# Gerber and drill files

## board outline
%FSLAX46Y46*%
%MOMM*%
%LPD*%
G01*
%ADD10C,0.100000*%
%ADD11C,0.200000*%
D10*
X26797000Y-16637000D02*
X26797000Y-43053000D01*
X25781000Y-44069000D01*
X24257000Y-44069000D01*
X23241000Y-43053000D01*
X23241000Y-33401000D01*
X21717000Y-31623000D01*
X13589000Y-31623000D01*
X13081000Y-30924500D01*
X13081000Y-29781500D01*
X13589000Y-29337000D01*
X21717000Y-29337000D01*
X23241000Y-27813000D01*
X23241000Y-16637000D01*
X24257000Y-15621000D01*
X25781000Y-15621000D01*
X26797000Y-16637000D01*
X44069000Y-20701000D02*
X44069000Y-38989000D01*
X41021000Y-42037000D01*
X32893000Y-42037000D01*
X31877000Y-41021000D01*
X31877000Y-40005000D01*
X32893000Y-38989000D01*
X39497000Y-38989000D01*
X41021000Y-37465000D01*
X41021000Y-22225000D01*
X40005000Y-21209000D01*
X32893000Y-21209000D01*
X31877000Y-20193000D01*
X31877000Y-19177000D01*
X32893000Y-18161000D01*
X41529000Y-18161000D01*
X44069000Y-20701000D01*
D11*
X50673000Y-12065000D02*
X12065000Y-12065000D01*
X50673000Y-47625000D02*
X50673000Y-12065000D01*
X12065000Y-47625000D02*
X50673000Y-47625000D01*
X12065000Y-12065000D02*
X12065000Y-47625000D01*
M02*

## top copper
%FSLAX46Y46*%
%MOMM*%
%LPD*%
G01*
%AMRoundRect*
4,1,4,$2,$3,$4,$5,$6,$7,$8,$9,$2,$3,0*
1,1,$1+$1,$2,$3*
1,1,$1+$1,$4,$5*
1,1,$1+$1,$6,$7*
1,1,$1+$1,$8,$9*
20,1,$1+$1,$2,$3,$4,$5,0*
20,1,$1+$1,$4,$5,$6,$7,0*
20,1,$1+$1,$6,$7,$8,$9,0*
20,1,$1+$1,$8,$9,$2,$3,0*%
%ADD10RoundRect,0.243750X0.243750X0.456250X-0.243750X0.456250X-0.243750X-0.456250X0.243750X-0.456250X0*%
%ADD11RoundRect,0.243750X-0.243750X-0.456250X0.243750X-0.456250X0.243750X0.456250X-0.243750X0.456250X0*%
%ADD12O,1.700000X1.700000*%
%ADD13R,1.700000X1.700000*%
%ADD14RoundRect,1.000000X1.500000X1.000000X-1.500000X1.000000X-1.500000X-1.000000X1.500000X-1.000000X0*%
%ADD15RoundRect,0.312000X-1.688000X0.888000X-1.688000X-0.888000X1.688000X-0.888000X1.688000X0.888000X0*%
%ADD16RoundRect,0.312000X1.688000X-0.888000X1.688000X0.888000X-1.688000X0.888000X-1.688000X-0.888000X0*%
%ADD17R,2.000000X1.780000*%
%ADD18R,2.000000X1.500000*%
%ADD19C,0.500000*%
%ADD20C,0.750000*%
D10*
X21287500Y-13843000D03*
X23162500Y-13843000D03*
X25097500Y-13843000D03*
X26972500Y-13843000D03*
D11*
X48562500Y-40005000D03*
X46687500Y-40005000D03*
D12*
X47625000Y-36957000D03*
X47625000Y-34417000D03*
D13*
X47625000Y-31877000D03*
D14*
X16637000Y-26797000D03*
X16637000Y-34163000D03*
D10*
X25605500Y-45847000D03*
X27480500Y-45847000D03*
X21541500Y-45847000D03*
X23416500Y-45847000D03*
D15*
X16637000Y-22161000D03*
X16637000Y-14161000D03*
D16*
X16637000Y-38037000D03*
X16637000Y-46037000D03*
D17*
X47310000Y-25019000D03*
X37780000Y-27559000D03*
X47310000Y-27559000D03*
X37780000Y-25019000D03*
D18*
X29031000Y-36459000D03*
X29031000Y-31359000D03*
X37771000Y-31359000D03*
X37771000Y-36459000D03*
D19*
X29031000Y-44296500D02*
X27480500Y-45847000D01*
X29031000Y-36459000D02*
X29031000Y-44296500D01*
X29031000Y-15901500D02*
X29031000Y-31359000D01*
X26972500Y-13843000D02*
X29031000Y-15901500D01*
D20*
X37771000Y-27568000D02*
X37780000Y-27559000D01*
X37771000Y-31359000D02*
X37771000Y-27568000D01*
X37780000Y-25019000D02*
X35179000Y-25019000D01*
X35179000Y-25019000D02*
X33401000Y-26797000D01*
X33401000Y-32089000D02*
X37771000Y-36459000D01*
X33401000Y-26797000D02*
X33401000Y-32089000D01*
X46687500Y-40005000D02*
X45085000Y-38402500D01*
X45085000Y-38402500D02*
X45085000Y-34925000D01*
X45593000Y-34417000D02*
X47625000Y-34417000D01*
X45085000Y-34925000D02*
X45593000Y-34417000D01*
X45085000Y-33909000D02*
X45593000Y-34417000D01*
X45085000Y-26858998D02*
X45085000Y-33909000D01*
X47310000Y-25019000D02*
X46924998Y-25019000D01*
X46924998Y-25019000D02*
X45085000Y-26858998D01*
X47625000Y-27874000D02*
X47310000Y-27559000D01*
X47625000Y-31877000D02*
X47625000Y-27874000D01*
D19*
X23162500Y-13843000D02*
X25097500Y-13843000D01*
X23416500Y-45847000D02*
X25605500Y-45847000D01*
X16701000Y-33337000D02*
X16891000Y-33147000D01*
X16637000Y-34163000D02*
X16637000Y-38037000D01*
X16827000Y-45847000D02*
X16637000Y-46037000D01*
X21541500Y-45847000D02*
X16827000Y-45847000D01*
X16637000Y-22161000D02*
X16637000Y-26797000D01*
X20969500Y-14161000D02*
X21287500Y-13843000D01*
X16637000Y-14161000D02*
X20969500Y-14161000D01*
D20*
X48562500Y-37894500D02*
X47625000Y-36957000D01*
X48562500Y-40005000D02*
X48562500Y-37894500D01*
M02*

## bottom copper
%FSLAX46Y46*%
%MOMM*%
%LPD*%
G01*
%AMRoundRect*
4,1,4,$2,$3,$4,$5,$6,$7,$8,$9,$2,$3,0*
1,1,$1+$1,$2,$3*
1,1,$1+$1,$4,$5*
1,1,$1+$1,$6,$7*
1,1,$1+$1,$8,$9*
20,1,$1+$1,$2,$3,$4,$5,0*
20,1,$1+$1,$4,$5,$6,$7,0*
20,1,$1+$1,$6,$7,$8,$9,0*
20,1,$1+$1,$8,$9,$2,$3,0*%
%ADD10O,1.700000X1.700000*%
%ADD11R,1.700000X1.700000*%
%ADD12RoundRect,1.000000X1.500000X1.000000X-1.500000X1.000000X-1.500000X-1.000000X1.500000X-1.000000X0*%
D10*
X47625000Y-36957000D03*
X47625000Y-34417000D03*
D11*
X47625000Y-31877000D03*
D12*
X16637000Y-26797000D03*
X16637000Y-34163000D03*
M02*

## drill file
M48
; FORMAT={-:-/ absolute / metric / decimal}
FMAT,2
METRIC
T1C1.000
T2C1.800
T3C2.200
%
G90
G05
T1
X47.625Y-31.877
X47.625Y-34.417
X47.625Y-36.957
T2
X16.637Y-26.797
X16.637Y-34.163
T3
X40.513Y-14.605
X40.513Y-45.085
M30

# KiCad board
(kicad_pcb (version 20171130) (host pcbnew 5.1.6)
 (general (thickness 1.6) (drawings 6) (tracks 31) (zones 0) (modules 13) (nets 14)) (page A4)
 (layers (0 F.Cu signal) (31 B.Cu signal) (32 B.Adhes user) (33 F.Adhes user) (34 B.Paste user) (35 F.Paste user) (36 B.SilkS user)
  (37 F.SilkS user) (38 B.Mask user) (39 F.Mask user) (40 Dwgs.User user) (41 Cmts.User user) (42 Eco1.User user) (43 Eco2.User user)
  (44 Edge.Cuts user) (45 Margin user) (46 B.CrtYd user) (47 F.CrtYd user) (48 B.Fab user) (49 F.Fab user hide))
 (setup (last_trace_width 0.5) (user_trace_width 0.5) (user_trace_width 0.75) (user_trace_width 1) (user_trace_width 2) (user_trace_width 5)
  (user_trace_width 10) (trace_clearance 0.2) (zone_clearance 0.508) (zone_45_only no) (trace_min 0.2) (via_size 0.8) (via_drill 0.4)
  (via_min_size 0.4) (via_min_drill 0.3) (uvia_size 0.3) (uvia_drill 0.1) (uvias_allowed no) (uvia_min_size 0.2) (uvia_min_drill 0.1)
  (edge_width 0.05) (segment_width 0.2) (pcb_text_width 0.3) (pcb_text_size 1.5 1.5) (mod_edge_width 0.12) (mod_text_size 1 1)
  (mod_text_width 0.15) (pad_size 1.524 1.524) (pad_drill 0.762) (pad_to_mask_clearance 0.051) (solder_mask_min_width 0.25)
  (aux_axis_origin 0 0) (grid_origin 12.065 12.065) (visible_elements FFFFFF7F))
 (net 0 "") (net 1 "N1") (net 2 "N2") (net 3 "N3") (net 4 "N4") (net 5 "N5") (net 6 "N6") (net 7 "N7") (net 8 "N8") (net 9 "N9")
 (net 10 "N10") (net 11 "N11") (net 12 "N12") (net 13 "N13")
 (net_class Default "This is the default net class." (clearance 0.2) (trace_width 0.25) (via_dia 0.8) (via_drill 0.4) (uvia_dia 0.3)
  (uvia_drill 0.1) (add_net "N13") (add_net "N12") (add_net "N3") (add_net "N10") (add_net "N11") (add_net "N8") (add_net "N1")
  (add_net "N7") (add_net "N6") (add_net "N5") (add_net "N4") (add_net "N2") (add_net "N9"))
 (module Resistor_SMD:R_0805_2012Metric (layer F.Cu) (at 22.225 13.843 180)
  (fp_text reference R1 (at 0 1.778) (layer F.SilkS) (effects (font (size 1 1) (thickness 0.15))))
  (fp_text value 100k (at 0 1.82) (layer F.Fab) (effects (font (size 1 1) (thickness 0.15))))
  (pad 2 smd roundrect (at 0.9375 0 180) (size 0.975 1.4) (layers F.Cu F.Paste F.Mask) (roundrect_rratio 0.25) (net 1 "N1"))
  (pad 1 smd roundrect (at -0.9375 0 180) (size 0.975 1.4) (layers F.Cu F.Paste F.Mask) (roundrect_rratio 0.25) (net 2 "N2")))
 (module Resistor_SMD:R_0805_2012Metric (layer F.Cu) (at 26.035 13.843 180)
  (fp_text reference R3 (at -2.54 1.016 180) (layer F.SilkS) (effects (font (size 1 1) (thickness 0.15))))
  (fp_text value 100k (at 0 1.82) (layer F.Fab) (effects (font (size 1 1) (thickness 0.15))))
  (pad 2 smd roundrect (at 0.9375 0 180) (size 0.975 1.4) (layers F.Cu F.Paste F.Mask) (roundrect_rratio 0.25) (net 2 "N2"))
  (pad 1 smd roundrect (at -0.9375 0 180) (size 0.975 1.4) (layers F.Cu F.Paste F.Mask) (roundrect_rratio 0.25) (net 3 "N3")))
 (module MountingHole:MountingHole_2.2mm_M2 (layer F.Cu) (at 40.513 45.085)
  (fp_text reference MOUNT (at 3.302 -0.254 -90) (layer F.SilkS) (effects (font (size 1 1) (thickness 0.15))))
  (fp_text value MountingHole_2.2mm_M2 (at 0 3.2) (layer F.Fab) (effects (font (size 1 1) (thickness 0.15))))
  (pad 1 np_thru_hole circle (at 0 0) (size 2.2 2.2) (drill 2.2) (layers *.Cu *.Mask)))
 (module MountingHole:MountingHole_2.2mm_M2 (layer F.Cu) (at 40.513 14.605)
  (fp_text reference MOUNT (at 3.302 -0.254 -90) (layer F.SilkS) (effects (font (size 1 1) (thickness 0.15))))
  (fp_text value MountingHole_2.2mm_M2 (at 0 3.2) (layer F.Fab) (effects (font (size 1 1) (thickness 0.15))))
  (pad 1 np_thru_hole circle (at 0 0) (size 2.2 2.2) (drill 2.2) (layers *.Cu *.Mask)))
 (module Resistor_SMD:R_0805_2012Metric (layer F.Cu) (at 47.625 40.005)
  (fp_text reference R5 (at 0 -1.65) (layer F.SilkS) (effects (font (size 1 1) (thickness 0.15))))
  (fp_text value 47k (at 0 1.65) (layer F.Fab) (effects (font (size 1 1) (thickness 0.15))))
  (pad 2 smd roundrect (at 0.9375 0) (size 0.975 1.4) (layers F.Cu F.Paste F.Mask) (roundrect_rratio 0.25) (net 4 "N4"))
  (pad 1 smd roundrect (at -0.9375 0) (size 0.975 1.4) (layers F.Cu F.Paste F.Mask) (roundrect_rratio 0.25) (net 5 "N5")))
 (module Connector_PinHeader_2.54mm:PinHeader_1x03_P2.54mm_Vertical (layer F.Cu) (at 47.625 31.877)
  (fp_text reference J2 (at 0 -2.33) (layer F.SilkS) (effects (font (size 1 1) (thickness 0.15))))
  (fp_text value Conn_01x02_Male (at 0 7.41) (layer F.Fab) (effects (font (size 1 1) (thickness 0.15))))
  (pad 3 thru_hole oval (at 0 5.08) (size 1.7 1.7) (drill 1) (layers *.Cu *.Mask) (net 4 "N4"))
  (pad 2 thru_hole oval (at 0 2.54) (size 1.7 1.7) (drill 1) (layers *.Cu *.Mask) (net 5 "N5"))
  (pad 1 thru_hole rect (at 0 0) (size 1.7 1.7) (drill 1) (layers *.Cu *.Mask) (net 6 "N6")))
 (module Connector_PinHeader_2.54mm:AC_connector (layer F.Cu) (at 16.637 34.417 180)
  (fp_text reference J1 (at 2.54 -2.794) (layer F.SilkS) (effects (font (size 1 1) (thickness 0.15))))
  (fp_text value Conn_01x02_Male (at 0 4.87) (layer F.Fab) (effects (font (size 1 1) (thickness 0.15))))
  (pad 2 thru_hole roundrect (at 0 7.62 180) (size 5 4) (drill 1.8) (layers *.Cu *.Mask) (roundrect_rratio 0.25) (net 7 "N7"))
  (pad 1 thru_hole roundrect (at 0 0.254 180) (size 5 4) (drill 1.8) (layers *.Cu *.Mask) (roundrect_rratio 0.25) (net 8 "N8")))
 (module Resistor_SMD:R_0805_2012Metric (layer F.Cu) (at 26.543 45.847 180)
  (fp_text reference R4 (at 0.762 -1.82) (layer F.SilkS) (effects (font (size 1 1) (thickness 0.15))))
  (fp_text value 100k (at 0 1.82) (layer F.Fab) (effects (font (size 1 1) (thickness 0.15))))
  (pad 2 smd roundrect (at 0.9375 0 180) (size 0.975 1.4) (layers F.Cu F.Paste F.Mask) (roundrect_rratio 0.25) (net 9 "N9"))
  (pad 1 smd roundrect (at -0.9375 0 180) (size 0.975 1.4) (layers F.Cu F.Paste F.Mask) (roundrect_rratio 0.25) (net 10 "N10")))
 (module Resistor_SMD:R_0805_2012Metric (layer F.Cu) (at 22.479 45.847 180)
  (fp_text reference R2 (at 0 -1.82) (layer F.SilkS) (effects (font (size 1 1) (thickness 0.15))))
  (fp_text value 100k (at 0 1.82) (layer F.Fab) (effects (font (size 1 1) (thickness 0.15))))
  (pad 2 smd roundrect (at 0.9375 0 180) (size 0.975 1.4) (layers F.Cu F.Paste F.Mask) (roundrect_rratio 0.25) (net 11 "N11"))
  (pad 1 smd roundrect (at -0.9375 0 180) (size 0.975 1.4) (layers F.Cu F.Paste F.Mask) (roundrect_rratio 0.25) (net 9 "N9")))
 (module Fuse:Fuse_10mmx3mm (layer F.Cu) (at 16.637 18.161 270)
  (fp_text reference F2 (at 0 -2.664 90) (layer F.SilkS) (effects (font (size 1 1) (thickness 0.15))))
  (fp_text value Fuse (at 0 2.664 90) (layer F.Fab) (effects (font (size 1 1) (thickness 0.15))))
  (pad 2 smd roundrect (at 4 0 270) (size 2.4 4) (layers F.Cu F.Paste F.Mask) (roundrect_rratio 0.13) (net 7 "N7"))
  (pad 1 smd roundrect (at -4 0 270) (size 2.4 4) (layers F.Cu F.Paste F.Mask) (roundrect_rratio 0.13) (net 1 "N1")))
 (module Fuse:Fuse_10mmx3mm (layer F.Cu) (at 16.637 42.037 90)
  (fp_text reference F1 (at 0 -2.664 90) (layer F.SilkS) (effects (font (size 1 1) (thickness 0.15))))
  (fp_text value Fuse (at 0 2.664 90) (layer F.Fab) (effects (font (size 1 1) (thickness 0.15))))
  (pad 2 smd roundrect (at 4 0 90) (size 2.4 4) (layers F.Cu F.Paste F.Mask) (roundrect_rratio 0.13) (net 8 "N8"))
  (pad 1 smd roundrect (at -4 0 90) (size 2.4 4) (layers F.Cu F.Paste F.Mask) (roundrect_rratio 0.13) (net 11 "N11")))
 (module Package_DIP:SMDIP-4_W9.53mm (layer F.Cu) (at 42.545 26.289)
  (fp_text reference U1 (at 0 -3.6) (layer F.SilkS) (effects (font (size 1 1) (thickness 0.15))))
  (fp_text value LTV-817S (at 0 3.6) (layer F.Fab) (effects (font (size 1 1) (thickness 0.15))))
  (pad 4 smd rect (at 4.765 -1.27) (size 2 1.78) (layers F.Cu F.Paste F.Mask) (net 5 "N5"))
  (pad 2 smd rect (at -4.765 1.27) (size 2 1.78) (layers F.Cu F.Paste F.Mask) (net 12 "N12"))
  (pad 3 smd rect (at 4.765 1.27) (size 2 1.78) (layers F.Cu F.Paste F.Mask) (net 6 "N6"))
  (pad 1 smd rect (at -4.765 -1.27) (size 2 1.78) (layers F.Cu F.Paste F.Mask) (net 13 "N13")))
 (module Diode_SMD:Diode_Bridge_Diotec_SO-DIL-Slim (layer F.Cu) (at 33.401 33.909 180)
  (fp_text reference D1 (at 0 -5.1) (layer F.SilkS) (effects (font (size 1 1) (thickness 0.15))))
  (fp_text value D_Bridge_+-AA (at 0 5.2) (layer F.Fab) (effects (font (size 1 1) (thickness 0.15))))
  (pad 4 smd rect (at 4.37 -2.55 180) (size 2 1.5) (layers F.Cu F.Paste F.Mask) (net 10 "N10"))
  (pad 3 smd rect (at 4.37 2.55 180) (size 2 1.5) (layers F.Cu F.Paste F.Mask) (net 3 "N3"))
  (pad 2 smd rect (at -4.37 2.55 180) (size 2 1.5) (layers F.Cu F.Paste F.Mask) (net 12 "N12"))
  (pad 1 smd rect (at -4.37 -2.55 180) (size 2 1.5) (layers F.Cu F.Paste F.Mask) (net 13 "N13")))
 (gr_poly
  (pts (xy 26.797 16.637) (xy 26.797 43.053) (xy 25.781 44.069) (xy 24.257 44.069) (xy 23.241 43.053) (xy 23.241 33.401) (xy 21.717 31.623)
   (xy 13.589 31.623) (xy 13.081 30.9245) (xy 13.081 29.7815) (xy 13.589 29.337) (xy 21.717 29.337) (xy 23.241 27.813) (xy 23.241 16.637)
   (xy 24.257 15.621) (xy 25.781 15.621))
  (layer Edge.Cuts) (width 0.1))
 (gr_poly
  (pts (xy 44.069 20.701) (xy 44.069 38.989) (xy 41.021 42.037) (xy 32.893 42.037) (xy 31.877 41.021) (xy 31.877 40.005) (xy 32.893 38.989)
   (xy 39.497 38.989) (xy 41.021 37.465) (xy 41.021 22.225) (xy 40.005 21.209) (xy 32.893 21.209) (xy 31.877 20.193) (xy 31.877 19.177)
   (xy 32.893 18.161) (xy 41.529 18.161))
  (layer Edge.Cuts) (width 0.1))
 (gr_line (start 50.673 12.065) (end 12.065 12.065) (layer Edge.Cuts) (width 0.2))
 (gr_line (start 50.673 47.625) (end 50.673 12.065) (layer Edge.Cuts) (width 0.2))
 (gr_line (start 12.065 47.625) (end 50.673 47.625) (layer Edge.Cuts) (width 0.2))
 (gr_line (start 12.065 12.065) (end 12.065 47.625) (layer Edge.Cuts) (width 0.2))
 (segment (start 29.031 44.2965) (end 27.4805 45.847) (width 0.5) (layer F.Cu) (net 10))
 (segment (start 29.031 36.459) (end 29.031 44.2965) (width 0.5) (layer F.Cu) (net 10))
 (segment (start 29.031 15.9015) (end 29.031 31.359) (width 0.5) (layer F.Cu) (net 3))
 (segment (start 26.9725 13.843) (end 29.031 15.9015) (width 0.5) (layer F.Cu) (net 3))
 (segment (start 37.771 27.568) (end 37.78 27.559) (width 0.75) (layer F.Cu) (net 12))
 (segment (start 37.771 31.359) (end 37.771 27.568) (width 0.75) (layer F.Cu) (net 12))
 (segment (start 37.78 25.019) (end 35.179 25.019) (width 0.75) (layer F.Cu) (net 13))
 (segment (start 35.179 25.019) (end 33.401 26.797) (width 0.75) (layer F.Cu) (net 13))
 (segment (start 33.401 32.089) (end 37.771 36.459) (width 0.75) (layer F.Cu) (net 13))
 (segment (start 33.401 26.797) (end 33.401 32.089) (width 0.75) (layer F.Cu) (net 13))
 (segment (start 46.6875 40.005) (end 45.085 38.4025) (width 0.75) (layer F.Cu) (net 5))
 (segment (start 45.085 38.4025) (end 45.085 34.925) (width 0.75) (layer F.Cu) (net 5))
 (segment (start 45.593 34.417) (end 47.625 34.417) (width 0.75) (layer F.Cu) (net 5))
 (segment (start 45.085 34.925) (end 45.593 34.417) (width 0.75) (layer F.Cu) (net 5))
 (segment (start 45.085 33.909) (end 45.593 34.417) (width 0.75) (layer F.Cu) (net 5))
 (segment (start 45.085 26.858998) (end 45.085 33.909) (width 0.75) (layer F.Cu) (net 5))
 (segment (start 47.31 25.019) (end 46.924998 25.019) (width 0.75) (layer F.Cu) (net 5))
 (segment (start 46.924998 25.019) (end 45.085 26.858998) (width 0.75) (layer F.Cu) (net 5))
 (segment (start 47.625 27.874) (end 47.31 27.559) (width 0.75) (layer F.Cu) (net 6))
 (segment (start 47.625 31.877) (end 47.625 27.874) (width 0.75) (layer F.Cu) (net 6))
 (segment (start 23.1625 13.843) (end 25.0975 13.843) (width 0.5) (layer F.Cu) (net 2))
 (segment (start 23.4165 45.847) (end 25.6055 45.847) (width 0.5) (layer F.Cu) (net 9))
 (segment (start 16.701 33.337) (end 16.891 33.147) (width 0.5) (layer F.Cu) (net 8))
 (segment (start 16.637 34.163) (end 16.637 38.037) (width 0.5) (layer F.Cu) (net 8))
 (segment (start 16.827 45.847) (end 16.637 46.037) (width 0.5) (layer F.Cu) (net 11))
 (segment (start 21.5415 45.847) (end 16.827 45.847) (width 0.5) (layer F.Cu) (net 11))
 (segment (start 16.637 22.161) (end 16.637 26.797) (width 0.5) (layer F.Cu) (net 7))
 (segment (start 20.9695 14.161) (end 21.2875 13.843) (width 0.5) (layer F.Cu) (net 1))
 (segment (start 16.637 14.161) (end 20.9695 14.161) (width 0.5) (layer F.Cu) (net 1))
 (segment (start 48.5625 37.8945) (end 47.625 36.957) (width 0.75) (layer F.Cu) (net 4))
 (segment (start 48.5625 40.005) (end 48.5625 37.8945) (width 0.75) (layer F.Cu) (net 4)))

